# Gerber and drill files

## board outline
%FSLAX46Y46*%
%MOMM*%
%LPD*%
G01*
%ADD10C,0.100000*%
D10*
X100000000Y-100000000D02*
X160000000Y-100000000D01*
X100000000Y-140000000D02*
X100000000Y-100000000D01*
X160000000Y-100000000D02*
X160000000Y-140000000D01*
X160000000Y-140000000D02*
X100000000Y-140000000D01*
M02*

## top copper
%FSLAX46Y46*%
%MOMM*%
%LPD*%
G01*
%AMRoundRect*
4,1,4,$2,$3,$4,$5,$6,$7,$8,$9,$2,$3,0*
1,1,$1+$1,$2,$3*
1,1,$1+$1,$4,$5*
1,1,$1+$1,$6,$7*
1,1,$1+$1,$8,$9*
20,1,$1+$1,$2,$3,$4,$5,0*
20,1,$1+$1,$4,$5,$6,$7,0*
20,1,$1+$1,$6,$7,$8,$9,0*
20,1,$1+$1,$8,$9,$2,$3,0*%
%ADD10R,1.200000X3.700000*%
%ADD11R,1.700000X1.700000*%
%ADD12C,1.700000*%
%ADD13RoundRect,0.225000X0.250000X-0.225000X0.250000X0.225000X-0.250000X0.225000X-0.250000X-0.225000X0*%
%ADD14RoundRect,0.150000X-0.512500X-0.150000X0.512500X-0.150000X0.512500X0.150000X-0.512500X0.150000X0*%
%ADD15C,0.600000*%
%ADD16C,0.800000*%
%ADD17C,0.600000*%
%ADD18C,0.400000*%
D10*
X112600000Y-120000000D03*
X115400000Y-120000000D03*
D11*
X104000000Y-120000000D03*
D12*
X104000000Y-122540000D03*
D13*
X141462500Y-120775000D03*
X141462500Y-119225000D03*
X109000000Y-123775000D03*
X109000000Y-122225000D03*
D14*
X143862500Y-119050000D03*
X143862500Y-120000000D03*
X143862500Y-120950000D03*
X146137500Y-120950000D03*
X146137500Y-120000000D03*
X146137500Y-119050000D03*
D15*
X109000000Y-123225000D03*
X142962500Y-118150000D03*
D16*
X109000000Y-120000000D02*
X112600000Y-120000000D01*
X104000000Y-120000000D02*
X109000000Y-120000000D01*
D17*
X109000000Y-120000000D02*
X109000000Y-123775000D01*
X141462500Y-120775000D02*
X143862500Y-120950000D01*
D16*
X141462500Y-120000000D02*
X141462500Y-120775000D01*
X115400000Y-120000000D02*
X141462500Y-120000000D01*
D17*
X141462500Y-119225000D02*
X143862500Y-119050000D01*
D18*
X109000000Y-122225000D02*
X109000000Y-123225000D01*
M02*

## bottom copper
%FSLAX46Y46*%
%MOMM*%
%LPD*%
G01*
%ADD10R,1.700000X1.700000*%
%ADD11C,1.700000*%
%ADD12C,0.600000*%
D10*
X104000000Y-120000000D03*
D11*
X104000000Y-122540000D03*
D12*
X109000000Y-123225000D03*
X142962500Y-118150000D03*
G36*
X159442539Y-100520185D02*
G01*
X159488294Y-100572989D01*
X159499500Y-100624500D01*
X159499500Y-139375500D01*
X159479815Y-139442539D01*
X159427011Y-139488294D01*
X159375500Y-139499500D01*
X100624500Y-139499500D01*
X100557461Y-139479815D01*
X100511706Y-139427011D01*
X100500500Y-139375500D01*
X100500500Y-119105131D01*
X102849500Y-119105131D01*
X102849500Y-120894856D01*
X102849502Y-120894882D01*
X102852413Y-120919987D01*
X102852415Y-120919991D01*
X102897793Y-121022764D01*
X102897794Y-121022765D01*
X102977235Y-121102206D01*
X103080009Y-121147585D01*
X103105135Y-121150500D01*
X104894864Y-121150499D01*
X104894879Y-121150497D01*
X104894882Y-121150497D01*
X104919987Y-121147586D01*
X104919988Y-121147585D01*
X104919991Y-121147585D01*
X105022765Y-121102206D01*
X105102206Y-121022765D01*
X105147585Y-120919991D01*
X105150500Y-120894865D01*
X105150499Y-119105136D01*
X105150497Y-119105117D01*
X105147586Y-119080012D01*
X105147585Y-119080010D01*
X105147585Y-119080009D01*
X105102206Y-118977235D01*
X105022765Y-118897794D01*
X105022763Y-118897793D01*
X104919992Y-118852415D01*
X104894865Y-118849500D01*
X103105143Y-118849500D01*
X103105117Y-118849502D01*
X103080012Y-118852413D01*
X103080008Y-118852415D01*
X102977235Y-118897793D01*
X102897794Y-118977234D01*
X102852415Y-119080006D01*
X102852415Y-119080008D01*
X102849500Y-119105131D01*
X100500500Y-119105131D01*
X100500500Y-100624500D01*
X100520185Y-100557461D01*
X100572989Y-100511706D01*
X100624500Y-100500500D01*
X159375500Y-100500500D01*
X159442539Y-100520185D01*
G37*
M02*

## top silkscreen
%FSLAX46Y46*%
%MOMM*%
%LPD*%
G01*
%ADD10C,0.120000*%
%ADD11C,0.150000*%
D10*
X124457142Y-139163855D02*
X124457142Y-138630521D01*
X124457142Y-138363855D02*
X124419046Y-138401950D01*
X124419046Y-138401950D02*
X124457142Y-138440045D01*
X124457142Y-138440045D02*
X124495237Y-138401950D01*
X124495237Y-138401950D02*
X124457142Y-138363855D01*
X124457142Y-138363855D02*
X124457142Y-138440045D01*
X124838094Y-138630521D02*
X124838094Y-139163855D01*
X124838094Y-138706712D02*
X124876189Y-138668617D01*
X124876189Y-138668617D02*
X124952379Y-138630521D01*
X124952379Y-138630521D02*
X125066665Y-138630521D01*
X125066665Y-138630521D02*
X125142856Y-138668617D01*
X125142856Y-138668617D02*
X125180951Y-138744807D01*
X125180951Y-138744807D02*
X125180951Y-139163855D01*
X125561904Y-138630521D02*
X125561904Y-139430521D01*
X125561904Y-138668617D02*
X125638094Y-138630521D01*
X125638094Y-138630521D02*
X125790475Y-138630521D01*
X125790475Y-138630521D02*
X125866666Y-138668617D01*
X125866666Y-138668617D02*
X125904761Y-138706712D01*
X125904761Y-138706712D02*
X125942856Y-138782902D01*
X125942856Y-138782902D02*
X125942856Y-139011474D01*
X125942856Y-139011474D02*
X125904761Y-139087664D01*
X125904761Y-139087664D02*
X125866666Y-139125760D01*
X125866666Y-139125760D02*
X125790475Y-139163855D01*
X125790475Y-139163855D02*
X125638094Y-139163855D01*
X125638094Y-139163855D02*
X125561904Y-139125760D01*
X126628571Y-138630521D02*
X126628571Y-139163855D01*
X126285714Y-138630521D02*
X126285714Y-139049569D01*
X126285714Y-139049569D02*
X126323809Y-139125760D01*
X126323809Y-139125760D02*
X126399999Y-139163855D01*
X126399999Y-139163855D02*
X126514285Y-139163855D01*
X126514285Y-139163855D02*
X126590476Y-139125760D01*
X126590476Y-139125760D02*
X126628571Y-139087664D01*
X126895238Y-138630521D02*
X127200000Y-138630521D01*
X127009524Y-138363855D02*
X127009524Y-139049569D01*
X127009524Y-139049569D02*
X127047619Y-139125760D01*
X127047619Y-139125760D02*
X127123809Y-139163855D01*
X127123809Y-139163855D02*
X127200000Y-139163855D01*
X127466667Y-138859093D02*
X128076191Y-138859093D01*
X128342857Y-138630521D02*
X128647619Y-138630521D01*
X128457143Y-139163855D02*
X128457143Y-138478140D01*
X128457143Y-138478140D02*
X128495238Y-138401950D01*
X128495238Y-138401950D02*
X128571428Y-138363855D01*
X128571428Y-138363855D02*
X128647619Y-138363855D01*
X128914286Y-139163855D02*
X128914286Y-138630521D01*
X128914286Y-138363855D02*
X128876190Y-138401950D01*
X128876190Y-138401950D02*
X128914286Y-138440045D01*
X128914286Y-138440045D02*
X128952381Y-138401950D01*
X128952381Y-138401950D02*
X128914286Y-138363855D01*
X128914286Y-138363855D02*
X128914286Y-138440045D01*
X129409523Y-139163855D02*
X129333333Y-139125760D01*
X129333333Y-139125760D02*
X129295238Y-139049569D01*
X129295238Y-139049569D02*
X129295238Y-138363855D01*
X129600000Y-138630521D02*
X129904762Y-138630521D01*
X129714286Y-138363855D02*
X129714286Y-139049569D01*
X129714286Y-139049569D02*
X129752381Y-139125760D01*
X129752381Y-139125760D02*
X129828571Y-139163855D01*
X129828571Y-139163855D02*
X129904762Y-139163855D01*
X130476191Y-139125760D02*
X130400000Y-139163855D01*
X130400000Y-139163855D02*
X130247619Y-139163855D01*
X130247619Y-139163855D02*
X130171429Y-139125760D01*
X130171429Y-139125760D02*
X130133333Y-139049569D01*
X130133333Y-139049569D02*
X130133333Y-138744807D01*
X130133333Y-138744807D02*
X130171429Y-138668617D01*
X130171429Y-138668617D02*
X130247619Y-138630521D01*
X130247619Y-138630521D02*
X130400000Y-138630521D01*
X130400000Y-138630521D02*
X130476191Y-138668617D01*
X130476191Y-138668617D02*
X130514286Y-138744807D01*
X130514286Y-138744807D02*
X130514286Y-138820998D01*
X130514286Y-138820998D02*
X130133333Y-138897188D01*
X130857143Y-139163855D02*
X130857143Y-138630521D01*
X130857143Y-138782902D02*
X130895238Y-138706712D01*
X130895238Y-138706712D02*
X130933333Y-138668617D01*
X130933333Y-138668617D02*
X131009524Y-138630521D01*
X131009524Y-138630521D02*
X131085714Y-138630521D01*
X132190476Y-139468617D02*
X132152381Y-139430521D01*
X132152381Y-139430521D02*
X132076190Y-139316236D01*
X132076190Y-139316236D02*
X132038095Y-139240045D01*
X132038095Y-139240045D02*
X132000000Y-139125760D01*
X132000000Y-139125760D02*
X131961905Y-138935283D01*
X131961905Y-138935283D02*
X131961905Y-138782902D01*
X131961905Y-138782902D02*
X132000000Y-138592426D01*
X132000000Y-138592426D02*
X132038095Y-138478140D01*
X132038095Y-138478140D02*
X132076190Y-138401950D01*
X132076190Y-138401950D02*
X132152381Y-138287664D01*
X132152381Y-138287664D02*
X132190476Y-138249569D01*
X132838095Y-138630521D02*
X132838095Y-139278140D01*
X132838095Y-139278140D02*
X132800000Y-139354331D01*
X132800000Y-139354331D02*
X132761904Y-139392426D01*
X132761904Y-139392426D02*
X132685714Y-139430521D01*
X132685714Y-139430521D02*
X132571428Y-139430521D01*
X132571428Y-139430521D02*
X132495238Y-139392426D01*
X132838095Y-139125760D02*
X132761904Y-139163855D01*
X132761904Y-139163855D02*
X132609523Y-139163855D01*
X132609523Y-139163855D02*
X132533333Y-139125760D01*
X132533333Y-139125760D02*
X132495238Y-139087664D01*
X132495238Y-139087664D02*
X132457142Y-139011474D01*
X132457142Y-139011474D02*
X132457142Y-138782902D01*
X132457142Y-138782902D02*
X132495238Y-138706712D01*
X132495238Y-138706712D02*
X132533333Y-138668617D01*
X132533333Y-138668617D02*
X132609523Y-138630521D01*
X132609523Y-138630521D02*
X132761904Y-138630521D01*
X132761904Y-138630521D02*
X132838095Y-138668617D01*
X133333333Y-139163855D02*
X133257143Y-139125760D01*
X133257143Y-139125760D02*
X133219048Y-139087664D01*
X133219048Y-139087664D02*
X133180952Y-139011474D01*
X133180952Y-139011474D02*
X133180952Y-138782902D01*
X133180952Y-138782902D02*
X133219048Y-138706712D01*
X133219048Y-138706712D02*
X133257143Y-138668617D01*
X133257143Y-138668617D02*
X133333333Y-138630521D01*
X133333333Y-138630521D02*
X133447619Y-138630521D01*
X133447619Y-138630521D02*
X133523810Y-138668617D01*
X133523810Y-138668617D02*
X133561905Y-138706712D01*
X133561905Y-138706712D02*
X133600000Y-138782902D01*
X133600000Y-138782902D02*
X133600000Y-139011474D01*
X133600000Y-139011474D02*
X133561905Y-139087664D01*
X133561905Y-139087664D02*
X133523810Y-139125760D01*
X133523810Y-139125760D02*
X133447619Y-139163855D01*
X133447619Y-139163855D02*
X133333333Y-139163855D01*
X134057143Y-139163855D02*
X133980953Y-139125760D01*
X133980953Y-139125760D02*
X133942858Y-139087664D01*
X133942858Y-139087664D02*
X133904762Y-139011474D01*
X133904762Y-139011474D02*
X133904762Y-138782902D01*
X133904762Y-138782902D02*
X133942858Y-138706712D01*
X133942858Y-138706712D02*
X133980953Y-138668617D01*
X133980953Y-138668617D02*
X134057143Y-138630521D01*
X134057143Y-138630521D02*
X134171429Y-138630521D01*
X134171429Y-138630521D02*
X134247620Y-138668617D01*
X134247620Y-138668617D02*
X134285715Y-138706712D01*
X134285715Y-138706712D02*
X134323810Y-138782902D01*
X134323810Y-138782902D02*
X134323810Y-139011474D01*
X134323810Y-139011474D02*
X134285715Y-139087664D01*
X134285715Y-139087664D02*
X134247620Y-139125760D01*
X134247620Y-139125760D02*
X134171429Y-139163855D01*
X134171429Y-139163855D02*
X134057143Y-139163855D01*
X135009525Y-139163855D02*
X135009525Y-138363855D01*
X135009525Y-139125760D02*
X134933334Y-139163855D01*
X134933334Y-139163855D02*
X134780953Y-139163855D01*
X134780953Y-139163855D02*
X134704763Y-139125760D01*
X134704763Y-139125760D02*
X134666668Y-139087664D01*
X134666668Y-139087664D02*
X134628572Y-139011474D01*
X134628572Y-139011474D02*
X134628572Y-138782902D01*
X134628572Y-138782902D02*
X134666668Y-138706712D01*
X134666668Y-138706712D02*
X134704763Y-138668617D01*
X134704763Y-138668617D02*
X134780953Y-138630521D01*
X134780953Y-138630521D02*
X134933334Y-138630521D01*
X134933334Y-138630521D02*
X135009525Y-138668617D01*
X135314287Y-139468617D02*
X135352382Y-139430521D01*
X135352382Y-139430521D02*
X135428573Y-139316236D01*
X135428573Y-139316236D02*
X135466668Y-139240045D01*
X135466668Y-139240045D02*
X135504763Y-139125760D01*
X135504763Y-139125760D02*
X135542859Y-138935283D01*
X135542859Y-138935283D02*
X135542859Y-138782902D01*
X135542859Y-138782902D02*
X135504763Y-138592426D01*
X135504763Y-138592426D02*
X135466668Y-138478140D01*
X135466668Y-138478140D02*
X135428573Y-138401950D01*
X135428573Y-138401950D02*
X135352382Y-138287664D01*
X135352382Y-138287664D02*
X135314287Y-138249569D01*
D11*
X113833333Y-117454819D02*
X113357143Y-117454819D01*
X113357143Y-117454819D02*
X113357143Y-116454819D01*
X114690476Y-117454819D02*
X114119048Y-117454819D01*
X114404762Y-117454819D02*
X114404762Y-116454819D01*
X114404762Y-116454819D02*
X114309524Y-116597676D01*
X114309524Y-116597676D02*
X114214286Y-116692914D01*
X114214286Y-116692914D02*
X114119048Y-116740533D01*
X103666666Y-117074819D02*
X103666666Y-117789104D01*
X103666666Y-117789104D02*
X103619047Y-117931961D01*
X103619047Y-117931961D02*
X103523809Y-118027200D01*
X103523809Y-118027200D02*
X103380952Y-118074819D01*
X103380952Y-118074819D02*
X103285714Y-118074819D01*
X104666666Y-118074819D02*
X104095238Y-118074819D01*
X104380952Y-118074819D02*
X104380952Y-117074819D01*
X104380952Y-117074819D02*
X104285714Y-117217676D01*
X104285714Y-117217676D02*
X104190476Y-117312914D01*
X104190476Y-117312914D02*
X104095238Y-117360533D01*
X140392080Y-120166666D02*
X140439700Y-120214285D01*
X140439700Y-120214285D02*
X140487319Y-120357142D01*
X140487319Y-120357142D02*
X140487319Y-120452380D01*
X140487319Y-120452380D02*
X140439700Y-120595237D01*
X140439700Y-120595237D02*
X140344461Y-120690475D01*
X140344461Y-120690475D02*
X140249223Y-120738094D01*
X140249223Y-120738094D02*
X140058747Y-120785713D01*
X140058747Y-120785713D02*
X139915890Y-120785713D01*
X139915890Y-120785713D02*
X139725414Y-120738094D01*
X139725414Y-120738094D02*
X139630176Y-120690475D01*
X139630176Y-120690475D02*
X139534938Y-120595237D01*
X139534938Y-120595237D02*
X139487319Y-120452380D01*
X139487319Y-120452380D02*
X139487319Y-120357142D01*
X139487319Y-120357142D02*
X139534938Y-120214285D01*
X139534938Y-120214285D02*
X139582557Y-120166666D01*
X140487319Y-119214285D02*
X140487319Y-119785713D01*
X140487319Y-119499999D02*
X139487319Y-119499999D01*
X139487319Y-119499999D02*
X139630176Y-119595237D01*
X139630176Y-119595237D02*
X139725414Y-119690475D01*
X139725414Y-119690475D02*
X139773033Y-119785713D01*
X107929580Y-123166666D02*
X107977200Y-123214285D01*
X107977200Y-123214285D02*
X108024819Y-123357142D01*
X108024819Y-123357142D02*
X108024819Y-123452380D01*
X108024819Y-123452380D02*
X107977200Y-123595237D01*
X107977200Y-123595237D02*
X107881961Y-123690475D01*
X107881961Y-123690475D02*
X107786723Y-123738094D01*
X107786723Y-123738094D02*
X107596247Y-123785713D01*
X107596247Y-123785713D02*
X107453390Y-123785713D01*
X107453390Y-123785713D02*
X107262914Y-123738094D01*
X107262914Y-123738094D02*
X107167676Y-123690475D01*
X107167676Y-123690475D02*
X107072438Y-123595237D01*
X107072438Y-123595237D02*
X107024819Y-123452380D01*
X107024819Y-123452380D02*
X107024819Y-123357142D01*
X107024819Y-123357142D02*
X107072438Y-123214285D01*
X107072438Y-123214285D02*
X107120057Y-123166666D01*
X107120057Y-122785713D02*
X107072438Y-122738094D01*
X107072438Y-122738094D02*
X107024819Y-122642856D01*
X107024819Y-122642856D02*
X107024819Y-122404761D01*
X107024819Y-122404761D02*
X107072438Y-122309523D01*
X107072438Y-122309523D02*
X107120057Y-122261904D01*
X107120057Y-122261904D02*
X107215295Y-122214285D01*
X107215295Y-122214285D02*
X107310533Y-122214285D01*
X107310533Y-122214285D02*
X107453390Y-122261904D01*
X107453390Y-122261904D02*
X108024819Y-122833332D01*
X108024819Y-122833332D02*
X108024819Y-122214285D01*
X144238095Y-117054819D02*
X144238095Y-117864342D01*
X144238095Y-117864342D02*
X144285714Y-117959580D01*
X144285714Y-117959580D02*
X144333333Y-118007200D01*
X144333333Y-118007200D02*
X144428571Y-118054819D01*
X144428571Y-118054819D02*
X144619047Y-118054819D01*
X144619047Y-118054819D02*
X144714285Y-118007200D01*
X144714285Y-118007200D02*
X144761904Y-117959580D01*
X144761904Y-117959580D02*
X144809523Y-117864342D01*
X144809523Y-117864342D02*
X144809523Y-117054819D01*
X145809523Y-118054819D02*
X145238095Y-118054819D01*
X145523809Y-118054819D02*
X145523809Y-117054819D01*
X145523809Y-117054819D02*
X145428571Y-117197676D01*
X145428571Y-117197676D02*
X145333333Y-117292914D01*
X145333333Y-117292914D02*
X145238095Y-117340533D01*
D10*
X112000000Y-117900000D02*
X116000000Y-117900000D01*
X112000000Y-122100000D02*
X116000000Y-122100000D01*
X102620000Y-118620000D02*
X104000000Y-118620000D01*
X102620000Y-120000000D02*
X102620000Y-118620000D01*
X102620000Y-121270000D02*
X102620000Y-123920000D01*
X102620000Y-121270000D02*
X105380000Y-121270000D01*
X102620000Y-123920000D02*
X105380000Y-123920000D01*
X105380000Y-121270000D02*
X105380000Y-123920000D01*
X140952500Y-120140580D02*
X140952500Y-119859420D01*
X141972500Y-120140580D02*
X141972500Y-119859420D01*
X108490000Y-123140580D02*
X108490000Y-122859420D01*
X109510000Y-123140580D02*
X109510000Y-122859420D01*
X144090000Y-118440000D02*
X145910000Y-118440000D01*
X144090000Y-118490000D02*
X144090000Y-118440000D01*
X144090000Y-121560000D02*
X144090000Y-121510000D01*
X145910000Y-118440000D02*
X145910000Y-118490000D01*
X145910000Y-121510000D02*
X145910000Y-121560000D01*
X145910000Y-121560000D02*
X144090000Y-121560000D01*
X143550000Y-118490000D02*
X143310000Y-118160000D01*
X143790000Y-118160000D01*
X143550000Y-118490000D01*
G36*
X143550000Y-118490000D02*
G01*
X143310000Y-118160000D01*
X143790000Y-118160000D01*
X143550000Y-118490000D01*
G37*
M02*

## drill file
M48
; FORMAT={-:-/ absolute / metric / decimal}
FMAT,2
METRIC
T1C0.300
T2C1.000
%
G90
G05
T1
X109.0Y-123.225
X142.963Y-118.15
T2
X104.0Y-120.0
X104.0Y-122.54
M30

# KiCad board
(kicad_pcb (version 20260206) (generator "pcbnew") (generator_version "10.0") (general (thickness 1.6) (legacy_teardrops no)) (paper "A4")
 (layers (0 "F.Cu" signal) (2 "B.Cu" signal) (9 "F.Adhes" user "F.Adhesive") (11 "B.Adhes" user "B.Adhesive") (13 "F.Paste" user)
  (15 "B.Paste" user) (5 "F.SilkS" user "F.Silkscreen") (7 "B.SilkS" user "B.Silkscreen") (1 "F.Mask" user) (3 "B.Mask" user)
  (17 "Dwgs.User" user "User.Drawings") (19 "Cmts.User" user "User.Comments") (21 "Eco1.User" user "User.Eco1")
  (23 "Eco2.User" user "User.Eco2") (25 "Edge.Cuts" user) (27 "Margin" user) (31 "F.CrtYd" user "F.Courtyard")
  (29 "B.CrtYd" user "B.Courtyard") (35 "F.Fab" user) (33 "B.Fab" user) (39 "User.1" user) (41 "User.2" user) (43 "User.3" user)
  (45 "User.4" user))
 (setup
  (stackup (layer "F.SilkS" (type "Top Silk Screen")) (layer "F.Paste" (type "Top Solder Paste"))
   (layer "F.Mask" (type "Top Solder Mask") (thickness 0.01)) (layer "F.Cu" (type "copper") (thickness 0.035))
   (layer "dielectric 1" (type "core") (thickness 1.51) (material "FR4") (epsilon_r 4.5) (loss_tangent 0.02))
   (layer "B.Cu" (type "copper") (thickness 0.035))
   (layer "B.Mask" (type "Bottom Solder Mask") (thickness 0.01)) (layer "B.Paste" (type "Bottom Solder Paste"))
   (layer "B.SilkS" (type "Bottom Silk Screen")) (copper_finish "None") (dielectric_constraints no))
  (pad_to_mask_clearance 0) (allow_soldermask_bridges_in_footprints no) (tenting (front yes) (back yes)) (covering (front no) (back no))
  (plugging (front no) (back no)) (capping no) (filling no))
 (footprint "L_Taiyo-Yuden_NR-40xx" (layer "F.Cu") (at 114 120)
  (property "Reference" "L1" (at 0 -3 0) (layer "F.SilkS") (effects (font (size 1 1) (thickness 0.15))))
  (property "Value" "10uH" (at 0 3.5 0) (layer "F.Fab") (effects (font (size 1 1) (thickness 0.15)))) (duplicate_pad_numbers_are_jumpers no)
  (fp_line (start -2 -2.1) (end 2 -2.1) (stroke (width 0.12) (type solid)) (layer "F.SilkS"))
  (fp_line (start -2 2.1) (end 2 2.1) (stroke (width 0.12) (type solid)) (layer "F.SilkS"))
  (pad "1" smd rect (at -1.4 0) (size 1.2 3.7) (layers "F.Cu" "F.Mask" "F.Paste") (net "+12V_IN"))
  (pad "2" smd rect (at 1.4 0) (size 1.2 3.7) (layers "F.Cu" "F.Mask" "F.Paste") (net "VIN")))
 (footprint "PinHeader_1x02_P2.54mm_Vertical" (layer "F.Cu") (at 104 120)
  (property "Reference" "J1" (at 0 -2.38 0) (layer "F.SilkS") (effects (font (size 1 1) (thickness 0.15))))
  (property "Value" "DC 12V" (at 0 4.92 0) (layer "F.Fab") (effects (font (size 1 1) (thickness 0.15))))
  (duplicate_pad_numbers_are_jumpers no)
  (fp_line (start -1.38 -1.38) (end 0 -1.38) (stroke (width 0.12) (type solid)) (layer "F.SilkS"))
  (fp_line (start -1.38 0) (end -1.38 -1.38) (stroke (width 0.12) (type solid)) (layer "F.SilkS"))
  (fp_line (start -1.38 1.27) (end -1.38 3.92) (stroke (width 0.12) (type solid)) (layer "F.SilkS"))
  (fp_line (start -1.38 1.27) (end 1.38 1.27) (stroke (width 0.12) (type solid)) (layer "F.SilkS"))
  (fp_line (start -1.38 3.92) (end 1.38 3.92) (stroke (width 0.12) (type solid)) (layer "F.SilkS"))
  (fp_line (start 1.38 1.27) (end 1.38 3.92) (stroke (width 0.12) (type solid)) (layer "F.SilkS"))
  (pad "1" thru_hole rect (at 0 0) (size 1.7 1.7) (drill 1) (layers "*.Cu" "*.Mask") (remove_unused_layers no) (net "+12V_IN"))
  (pad "2" thru_hole circle (at 0 2.54) (size 1.7 1.7) (drill 1) (layers "*.Cu" "*.Mask") (remove_unused_layers no) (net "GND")))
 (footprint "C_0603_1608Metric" (layer "F.Cu") (at 141.4625 120 90)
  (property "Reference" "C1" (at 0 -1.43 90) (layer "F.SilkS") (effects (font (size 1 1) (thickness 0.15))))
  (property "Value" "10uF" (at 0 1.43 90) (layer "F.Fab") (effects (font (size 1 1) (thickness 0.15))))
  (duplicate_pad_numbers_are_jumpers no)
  (fp_line (start -0.14058 -0.51) (end 0.14058 -0.51) (stroke (width 0.12) (type solid)) (layer "F.SilkS"))
  (fp_line (start -0.14058 0.51) (end 0.14058 0.51) (stroke (width 0.12) (type solid)) (layer "F.SilkS"))
  (pad "1" smd roundrect (at -0.775 0 90) (size 0.9 0.95) (layers "F.Cu" "F.Mask" "F.Paste") (roundrect_rratio 0.25) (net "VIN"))
  (pad "2" smd roundrect (at 0.775 0 90) (size 0.9 0.95) (layers "F.Cu" "F.Mask" "F.Paste") (roundrect_rratio 0.25) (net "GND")))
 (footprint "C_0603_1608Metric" (layer "F.Cu") (at 109 123 90)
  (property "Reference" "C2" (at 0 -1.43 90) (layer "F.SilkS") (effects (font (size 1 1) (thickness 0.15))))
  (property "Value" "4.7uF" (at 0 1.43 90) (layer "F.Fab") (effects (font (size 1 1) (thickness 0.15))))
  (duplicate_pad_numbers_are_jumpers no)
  (fp_line (start -0.14058 -0.51) (end 0.14058 -0.51) (stroke (width 0.12) (type solid)) (layer "F.SilkS"))
  (fp_line (start -0.14058 0.51) (end 0.14058 0.51) (stroke (width 0.12) (type solid)) (layer "F.SilkS"))
  (pad "1" smd roundrect (at -0.775 0 90) (size 0.9 0.95) (layers "F.Cu" "F.Mask" "F.Paste") (roundrect_rratio 0.25) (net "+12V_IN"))
  (pad "2" smd roundrect (at 0.775 0 90) (size 0.9 0.95) (layers "F.Cu" "F.Mask" "F.Paste") (roundrect_rratio 0.25) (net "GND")))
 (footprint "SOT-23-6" (layer "F.Cu") (at 145 120)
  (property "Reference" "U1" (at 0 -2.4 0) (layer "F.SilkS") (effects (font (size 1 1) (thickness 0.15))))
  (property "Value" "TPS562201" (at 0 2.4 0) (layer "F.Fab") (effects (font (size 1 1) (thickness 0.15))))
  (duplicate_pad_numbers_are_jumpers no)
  (fp_line (start -0.91 -1.56) (end 0.91 -1.56) (stroke (width 0.12) (type solid)) (layer "F.SilkS"))
  (fp_line (start -0.91 -1.51) (end -0.91 -1.56) (stroke (width 0.12) (type solid)) (layer "F.SilkS"))
  (fp_line (start -0.91 1.56) (end -0.91 1.51) (stroke (width 0.12) (type solid)) (layer "F.SilkS"))
  (fp_line (start 0.91 -1.56) (end 0.91 -1.51) (stroke (width 0.12) (type solid)) (layer "F.SilkS"))
  (fp_line (start 0.91 1.51) (end 0.91 1.56) (stroke (width 0.12) (type solid)) (layer "F.SilkS"))
  (fp_line (start 0.91 1.56) (end -0.91 1.56) (stroke (width 0.12) (type solid)) (layer "F.SilkS"))
  (fp_poly (pts (xy -1.45 -1.51) (xy -1.69 -1.84) (xy -1.21 -1.84)) (stroke (width 0.12) (type solid)) (fill yes) (layer "F.SilkS"))
  (pad "1" smd roundrect (at -1.1375 -0.95) (size 1.325 0.6) (layers "F.Cu" "F.Mask" "F.Paste") (roundrect_rratio 0.25) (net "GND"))
  (pad "2" smd roundrect (at -1.1375 0) (size 1.325 0.6) (layers "F.Cu" "F.Mask" "F.Paste") (roundrect_rratio 0.25) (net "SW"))
  (pad "3" smd roundrect (at -1.1375 0.95) (size 1.325 0.6) (layers "F.Cu" "F.Mask" "F.Paste") (roundrect_rratio 0.25) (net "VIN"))
  (pad "4" smd roundrect (at 1.1375 0.95) (size 1.325 0.6) (layers "F.Cu" "F.Mask" "F.Paste") (roundrect_rratio 0.25) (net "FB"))
  (pad "5" smd roundrect (at 1.1375 0) (size 1.325 0.6) (layers "F.Cu" "F.Mask" "F.Paste") (roundrect_rratio 0.25) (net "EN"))
  (pad "6" smd roundrect (at 1.1375 -0.95) (size 1.325 0.6) (layers "F.Cu" "F.Mask" "F.Paste") (roundrect_rratio 0.25) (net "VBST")))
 (gr_line (start 100 100) (end 160 100) (stroke (width 0.1) (type default)) (layer "Edge.Cuts"))
 (gr_line (start 100 140) (end 100 100) (stroke (width 0.1) (type default)) (layer "Edge.Cuts"))
 (gr_line (start 160 100) (end 160 140) (stroke (width 0.1) (type default)) (layer "Edge.Cuts"))
 (gr_line (start 160 140) (end 100 140) (stroke (width 0.1) (type default)) (layer "Edge.Cuts"))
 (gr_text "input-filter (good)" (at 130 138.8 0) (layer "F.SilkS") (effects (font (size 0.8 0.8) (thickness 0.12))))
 (segment (start 109 120) (end 112.6 120) (width 0.8) (layer "F.Cu") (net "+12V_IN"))
 (segment (start 104 120) (end 109 120) (width 0.8) (layer "F.Cu") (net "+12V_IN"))
 (segment (start 109 120) (end 109 123.775) (width 0.6) (layer "F.Cu") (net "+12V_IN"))
 (segment (start 141.4625 120.775) (end 143.8625 120.95) (width 0.6) (layer "F.Cu") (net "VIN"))
 (segment (start 141.4625 120) (end 141.4625 120.775) (width 0.8) (layer "F.Cu") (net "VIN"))
 (segment (start 115.4 120) (end 141.4625 120) (width 0.8) (layer "F.Cu") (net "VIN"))
 (segment (start 141.4625 119.225) (end 143.8625 119.05) (width 0.6) (layer "F.Cu") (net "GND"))
 (segment (start 109 122.225) (end 109 123.225) (width 0.4) (layer "F.Cu") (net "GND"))
 (via (at 109 123.225) (size 0.6) (drill 0.3) (layers "F.Cu" "B.Cu") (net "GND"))
 (via (at 142.9625 118.15) (size 0.6) (drill 0.3) (layers "F.Cu" "B.Cu") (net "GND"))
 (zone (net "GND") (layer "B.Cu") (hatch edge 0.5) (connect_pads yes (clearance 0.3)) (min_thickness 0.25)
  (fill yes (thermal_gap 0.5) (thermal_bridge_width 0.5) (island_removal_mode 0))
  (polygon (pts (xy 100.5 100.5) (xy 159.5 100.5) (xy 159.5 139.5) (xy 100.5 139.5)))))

